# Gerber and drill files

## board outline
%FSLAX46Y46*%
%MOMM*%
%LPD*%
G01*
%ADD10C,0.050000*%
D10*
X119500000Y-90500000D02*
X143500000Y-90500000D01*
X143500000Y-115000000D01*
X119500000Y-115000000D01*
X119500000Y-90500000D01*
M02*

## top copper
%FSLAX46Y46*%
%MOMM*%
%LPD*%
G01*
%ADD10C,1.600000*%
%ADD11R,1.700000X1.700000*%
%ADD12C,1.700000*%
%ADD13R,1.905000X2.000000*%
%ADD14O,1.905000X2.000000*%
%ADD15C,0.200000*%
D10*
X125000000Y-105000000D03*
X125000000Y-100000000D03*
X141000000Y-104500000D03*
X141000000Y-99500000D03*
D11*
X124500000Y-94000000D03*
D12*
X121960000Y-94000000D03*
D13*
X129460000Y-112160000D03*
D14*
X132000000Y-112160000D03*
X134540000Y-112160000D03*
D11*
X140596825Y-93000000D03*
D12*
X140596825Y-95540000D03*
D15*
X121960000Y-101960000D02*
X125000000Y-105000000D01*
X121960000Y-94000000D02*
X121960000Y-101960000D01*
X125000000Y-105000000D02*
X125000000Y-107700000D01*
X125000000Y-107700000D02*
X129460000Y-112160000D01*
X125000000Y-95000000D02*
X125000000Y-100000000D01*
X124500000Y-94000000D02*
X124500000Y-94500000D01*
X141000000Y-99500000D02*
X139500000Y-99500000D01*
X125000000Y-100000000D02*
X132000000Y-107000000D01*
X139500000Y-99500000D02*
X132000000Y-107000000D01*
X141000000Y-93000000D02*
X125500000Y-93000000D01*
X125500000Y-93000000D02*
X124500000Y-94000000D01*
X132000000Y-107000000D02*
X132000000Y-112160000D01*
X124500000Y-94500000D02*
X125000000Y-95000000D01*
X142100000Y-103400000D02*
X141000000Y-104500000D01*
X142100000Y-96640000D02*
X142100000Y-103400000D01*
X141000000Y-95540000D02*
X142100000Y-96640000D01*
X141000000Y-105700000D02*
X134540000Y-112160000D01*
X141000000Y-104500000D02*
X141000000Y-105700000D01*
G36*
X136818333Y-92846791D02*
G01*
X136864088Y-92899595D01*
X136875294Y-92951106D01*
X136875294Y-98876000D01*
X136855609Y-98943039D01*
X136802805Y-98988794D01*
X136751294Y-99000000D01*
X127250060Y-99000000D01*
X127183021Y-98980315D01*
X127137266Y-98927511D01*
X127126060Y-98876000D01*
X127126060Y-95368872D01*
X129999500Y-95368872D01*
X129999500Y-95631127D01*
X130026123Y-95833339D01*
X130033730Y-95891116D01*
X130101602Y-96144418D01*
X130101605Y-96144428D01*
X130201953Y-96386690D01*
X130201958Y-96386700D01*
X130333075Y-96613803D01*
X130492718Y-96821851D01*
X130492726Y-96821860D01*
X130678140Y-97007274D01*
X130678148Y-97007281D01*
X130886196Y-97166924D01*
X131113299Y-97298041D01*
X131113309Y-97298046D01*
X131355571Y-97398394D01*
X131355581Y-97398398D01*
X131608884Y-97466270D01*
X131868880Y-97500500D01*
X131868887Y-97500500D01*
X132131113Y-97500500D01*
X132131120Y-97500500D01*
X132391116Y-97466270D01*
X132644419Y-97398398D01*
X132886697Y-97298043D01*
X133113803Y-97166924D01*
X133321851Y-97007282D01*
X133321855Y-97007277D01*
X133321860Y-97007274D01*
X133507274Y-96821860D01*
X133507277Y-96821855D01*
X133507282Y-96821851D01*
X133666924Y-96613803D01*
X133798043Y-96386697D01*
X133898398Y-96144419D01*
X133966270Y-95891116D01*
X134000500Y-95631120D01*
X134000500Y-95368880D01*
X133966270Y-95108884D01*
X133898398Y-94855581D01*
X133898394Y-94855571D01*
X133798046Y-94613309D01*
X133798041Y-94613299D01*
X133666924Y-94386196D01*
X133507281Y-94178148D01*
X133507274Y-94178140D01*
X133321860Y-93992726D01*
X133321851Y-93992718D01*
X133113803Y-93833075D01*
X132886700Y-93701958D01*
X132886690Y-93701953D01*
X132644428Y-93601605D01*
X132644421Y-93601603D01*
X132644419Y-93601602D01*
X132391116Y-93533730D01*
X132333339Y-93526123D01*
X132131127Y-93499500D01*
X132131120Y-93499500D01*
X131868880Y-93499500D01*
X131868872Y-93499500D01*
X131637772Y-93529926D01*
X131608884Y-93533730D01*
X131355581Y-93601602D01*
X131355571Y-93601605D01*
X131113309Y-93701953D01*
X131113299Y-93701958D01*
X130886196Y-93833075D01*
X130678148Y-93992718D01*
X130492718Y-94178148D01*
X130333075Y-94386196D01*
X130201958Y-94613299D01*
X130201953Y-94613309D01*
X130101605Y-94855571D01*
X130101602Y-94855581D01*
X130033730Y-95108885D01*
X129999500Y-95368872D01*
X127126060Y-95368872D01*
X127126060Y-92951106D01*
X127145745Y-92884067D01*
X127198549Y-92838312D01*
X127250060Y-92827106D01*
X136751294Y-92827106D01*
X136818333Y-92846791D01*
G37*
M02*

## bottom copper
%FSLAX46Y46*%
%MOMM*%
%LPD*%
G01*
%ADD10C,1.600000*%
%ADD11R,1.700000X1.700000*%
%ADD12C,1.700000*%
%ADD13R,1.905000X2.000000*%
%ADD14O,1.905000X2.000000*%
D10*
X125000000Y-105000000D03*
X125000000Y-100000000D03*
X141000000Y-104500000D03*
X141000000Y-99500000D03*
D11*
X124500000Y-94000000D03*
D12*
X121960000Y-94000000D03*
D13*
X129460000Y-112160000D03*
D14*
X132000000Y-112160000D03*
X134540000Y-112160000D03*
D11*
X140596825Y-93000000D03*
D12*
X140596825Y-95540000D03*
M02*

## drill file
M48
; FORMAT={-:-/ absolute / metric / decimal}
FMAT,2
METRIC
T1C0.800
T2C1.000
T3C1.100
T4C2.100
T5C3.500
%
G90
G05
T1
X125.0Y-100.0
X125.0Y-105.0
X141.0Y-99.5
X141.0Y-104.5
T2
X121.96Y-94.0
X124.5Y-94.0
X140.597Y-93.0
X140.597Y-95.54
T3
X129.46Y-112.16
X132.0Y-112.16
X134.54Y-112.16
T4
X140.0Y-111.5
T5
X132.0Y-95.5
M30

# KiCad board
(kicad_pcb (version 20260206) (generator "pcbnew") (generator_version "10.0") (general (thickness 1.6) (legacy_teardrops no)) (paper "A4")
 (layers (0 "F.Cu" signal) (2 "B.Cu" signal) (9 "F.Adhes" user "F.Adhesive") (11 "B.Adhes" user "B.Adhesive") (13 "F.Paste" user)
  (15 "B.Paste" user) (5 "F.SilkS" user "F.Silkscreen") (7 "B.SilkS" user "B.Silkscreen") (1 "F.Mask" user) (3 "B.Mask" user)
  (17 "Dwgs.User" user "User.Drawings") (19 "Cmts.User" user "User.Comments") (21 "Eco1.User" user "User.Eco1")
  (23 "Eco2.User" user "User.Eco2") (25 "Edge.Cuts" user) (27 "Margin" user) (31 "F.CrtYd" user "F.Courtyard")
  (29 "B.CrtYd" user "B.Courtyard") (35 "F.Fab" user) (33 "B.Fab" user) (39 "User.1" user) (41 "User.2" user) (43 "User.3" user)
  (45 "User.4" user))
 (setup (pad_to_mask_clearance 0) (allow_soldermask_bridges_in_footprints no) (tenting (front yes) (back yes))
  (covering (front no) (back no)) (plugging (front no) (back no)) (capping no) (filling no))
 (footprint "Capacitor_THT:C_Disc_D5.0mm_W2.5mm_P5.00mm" (layer "F.Cu") (at 125 105 90)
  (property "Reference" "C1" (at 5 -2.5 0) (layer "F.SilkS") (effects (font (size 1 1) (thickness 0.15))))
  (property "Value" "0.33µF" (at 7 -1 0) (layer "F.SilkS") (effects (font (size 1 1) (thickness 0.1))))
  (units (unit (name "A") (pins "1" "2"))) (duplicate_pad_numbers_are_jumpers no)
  (pad "1" thru_hole circle (at 0 0 90) (size 1.6 1.6) (drill 0.8) (layers "*.Cu" "*.Mask") (remove_unused_layers no) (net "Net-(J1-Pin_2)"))
  (pad "2" thru_hole circle (at 5 0 90) (size 1.6 1.6) (drill 0.8) (layers "*.Cu" "*.Mask") (remove_unused_layers no) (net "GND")))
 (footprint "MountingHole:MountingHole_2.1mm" (layer "F.Cu") (at 140 111.5)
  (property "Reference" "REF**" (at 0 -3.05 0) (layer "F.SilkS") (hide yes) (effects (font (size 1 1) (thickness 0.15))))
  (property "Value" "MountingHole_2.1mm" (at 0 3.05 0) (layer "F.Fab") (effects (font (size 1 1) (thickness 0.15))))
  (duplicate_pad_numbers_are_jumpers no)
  (pad "" np_thru_hole circle (at 0 0) (size 2.1 2.1) (drill 2.1) (layers "*.Cu" "*.Mask")))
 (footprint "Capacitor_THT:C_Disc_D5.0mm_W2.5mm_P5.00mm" (layer "F.Cu") (at 141 104.5 90)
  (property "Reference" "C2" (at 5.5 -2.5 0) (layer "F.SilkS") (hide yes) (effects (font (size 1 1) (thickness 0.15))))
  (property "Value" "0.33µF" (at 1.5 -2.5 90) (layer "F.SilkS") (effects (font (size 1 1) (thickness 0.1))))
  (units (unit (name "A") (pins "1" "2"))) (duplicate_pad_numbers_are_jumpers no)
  (pad "1" thru_hole circle (at 0 0 90) (size 1.6 1.6) (drill 0.8) (layers "*.Cu" "*.Mask") (remove_unused_layers no) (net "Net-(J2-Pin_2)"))
  (pad "2" thru_hole circle (at 5 0 90) (size 1.6 1.6) (drill 0.8) (layers "*.Cu" "*.Mask") (remove_unused_layers no) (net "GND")))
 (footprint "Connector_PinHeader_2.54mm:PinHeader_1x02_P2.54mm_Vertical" (layer "F.Cu") (at 124.5 94 -90)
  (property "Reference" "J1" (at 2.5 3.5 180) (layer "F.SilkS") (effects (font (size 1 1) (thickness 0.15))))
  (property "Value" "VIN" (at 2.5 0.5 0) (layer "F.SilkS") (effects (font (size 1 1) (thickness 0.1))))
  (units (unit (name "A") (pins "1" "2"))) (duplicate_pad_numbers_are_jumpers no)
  (pad "1" thru_hole rect (at 0 0 270) (size 1.7 1.7) (drill 1) (layers "*.Cu" "*.Mask") (remove_unused_layers no) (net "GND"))
  (pad "2" thru_hole circle (at 0 2.54 270) (size 1.7 1.7) (drill 1) (layers "*.Cu" "*.Mask") (remove_unused_layers no)
   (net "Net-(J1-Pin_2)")))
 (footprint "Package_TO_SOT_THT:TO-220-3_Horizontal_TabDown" (layer "F.Cu") (at 129.46 112.16)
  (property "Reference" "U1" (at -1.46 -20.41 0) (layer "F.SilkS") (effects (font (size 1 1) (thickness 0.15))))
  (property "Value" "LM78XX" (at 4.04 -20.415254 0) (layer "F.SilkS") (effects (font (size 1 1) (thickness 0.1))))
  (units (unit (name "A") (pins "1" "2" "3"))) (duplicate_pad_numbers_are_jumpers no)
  (pad "" np_thru_hole circle (at 2.54 -16.66) (size 3.5 3.5) (drill 3.5) (layers "*.Cu" "*.Mask"))
  (pad "1" thru_hole rect (at 0 0) (size 1.905 2) (drill 1.1) (layers "*.Cu" "*.Mask") (remove_unused_layers no) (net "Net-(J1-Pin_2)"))
  (pad "2" thru_hole oval (at 2.54 0) (size 1.905 2) (drill 1.1) (layers "*.Cu" "*.Mask") (remove_unused_layers no) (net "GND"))
  (pad "3" thru_hole oval (at 5.08 0) (size 1.905 2) (drill 1.1) (layers "*.Cu" "*.Mask") (remove_unused_layers no) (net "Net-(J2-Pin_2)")))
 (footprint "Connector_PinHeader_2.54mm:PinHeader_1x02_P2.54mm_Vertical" (layer "F.Cu") (at 140.596825 93)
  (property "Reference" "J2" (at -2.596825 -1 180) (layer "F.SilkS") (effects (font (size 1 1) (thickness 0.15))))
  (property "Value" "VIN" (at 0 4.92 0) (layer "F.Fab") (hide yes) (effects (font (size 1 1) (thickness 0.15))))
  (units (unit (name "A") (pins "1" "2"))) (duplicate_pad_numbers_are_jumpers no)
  (pad "1" thru_hole rect (at 0 0) (size 1.7 1.7) (drill 1) (layers "*.Cu" "*.Mask") (remove_unused_layers no) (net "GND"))
  (pad "2" thru_hole circle (at 0 2.54) (size 1.7 1.7) (drill 1) (layers "*.Cu" "*.Mask") (remove_unused_layers no) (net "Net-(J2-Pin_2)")))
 (gr_rect (start 119.5 90.5) (end 143.5 115) (stroke (width 0.05) (type default)) (fill no) (layer "Edge.Cuts"))
 (segment (start 121.96 101.96) (end 125 105) (width 0.2) (layer "F.Cu") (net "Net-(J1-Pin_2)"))
 (segment (start 121.96 94) (end 121.96 101.96) (width 0.2) (layer "F.Cu") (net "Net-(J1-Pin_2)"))
 (segment (start 125 105) (end 125 107.7) (width 0.2) (layer "F.Cu") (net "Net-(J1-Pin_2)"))
 (segment (start 125 107.7) (end 129.46 112.16) (width 0.2) (layer "F.Cu") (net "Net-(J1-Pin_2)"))
 (segment (start 125 95) (end 125 100) (width 0.2) (layer "F.Cu") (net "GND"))
 (segment (start 124.5 94) (end 124.5 94.5) (width 0.2) (layer "F.Cu") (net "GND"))
 (segment (start 141 99.5) (end 139.5 99.5) (width 0.2) (layer "F.Cu") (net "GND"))
 (segment (start 125 100) (end 132 107) (width 0.2) (layer "F.Cu") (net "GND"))
 (segment (start 139.5 99.5) (end 132 107) (width 0.2) (layer "F.Cu") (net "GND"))
 (segment (start 141 93) (end 125.5 93) (width 0.2) (layer "F.Cu") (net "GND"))
 (segment (start 125.5 93) (end 124.5 94) (width 0.2) (layer "F.Cu") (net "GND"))
 (segment (start 132 107) (end 132 112.16) (width 0.2) (layer "F.Cu") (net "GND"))
 (segment (start 124.5 94.5) (end 125 95) (width 0.2) (layer "F.Cu") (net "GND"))
 (segment (start 142.1 103.4) (end 141 104.5) (width 0.2) (layer "F.Cu") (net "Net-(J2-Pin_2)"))
 (segment (start 142.1 96.64) (end 142.1 103.4) (width 0.2) (layer "F.Cu") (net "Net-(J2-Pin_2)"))
 (segment (start 141 95.54) (end 142.1 96.64) (width 0.2) (layer "F.Cu") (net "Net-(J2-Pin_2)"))
 (segment (start 141 105.7) (end 134.54 112.16) (width 0.2) (layer "F.Cu") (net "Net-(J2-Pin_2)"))
 (segment (start 141 104.5) (end 141 105.7) (width 0.2) (layer "F.Cu") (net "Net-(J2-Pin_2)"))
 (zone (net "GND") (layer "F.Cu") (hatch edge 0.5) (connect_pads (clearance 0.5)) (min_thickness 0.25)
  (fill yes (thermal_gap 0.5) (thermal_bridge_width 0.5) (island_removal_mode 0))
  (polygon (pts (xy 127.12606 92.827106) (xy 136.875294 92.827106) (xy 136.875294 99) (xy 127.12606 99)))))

